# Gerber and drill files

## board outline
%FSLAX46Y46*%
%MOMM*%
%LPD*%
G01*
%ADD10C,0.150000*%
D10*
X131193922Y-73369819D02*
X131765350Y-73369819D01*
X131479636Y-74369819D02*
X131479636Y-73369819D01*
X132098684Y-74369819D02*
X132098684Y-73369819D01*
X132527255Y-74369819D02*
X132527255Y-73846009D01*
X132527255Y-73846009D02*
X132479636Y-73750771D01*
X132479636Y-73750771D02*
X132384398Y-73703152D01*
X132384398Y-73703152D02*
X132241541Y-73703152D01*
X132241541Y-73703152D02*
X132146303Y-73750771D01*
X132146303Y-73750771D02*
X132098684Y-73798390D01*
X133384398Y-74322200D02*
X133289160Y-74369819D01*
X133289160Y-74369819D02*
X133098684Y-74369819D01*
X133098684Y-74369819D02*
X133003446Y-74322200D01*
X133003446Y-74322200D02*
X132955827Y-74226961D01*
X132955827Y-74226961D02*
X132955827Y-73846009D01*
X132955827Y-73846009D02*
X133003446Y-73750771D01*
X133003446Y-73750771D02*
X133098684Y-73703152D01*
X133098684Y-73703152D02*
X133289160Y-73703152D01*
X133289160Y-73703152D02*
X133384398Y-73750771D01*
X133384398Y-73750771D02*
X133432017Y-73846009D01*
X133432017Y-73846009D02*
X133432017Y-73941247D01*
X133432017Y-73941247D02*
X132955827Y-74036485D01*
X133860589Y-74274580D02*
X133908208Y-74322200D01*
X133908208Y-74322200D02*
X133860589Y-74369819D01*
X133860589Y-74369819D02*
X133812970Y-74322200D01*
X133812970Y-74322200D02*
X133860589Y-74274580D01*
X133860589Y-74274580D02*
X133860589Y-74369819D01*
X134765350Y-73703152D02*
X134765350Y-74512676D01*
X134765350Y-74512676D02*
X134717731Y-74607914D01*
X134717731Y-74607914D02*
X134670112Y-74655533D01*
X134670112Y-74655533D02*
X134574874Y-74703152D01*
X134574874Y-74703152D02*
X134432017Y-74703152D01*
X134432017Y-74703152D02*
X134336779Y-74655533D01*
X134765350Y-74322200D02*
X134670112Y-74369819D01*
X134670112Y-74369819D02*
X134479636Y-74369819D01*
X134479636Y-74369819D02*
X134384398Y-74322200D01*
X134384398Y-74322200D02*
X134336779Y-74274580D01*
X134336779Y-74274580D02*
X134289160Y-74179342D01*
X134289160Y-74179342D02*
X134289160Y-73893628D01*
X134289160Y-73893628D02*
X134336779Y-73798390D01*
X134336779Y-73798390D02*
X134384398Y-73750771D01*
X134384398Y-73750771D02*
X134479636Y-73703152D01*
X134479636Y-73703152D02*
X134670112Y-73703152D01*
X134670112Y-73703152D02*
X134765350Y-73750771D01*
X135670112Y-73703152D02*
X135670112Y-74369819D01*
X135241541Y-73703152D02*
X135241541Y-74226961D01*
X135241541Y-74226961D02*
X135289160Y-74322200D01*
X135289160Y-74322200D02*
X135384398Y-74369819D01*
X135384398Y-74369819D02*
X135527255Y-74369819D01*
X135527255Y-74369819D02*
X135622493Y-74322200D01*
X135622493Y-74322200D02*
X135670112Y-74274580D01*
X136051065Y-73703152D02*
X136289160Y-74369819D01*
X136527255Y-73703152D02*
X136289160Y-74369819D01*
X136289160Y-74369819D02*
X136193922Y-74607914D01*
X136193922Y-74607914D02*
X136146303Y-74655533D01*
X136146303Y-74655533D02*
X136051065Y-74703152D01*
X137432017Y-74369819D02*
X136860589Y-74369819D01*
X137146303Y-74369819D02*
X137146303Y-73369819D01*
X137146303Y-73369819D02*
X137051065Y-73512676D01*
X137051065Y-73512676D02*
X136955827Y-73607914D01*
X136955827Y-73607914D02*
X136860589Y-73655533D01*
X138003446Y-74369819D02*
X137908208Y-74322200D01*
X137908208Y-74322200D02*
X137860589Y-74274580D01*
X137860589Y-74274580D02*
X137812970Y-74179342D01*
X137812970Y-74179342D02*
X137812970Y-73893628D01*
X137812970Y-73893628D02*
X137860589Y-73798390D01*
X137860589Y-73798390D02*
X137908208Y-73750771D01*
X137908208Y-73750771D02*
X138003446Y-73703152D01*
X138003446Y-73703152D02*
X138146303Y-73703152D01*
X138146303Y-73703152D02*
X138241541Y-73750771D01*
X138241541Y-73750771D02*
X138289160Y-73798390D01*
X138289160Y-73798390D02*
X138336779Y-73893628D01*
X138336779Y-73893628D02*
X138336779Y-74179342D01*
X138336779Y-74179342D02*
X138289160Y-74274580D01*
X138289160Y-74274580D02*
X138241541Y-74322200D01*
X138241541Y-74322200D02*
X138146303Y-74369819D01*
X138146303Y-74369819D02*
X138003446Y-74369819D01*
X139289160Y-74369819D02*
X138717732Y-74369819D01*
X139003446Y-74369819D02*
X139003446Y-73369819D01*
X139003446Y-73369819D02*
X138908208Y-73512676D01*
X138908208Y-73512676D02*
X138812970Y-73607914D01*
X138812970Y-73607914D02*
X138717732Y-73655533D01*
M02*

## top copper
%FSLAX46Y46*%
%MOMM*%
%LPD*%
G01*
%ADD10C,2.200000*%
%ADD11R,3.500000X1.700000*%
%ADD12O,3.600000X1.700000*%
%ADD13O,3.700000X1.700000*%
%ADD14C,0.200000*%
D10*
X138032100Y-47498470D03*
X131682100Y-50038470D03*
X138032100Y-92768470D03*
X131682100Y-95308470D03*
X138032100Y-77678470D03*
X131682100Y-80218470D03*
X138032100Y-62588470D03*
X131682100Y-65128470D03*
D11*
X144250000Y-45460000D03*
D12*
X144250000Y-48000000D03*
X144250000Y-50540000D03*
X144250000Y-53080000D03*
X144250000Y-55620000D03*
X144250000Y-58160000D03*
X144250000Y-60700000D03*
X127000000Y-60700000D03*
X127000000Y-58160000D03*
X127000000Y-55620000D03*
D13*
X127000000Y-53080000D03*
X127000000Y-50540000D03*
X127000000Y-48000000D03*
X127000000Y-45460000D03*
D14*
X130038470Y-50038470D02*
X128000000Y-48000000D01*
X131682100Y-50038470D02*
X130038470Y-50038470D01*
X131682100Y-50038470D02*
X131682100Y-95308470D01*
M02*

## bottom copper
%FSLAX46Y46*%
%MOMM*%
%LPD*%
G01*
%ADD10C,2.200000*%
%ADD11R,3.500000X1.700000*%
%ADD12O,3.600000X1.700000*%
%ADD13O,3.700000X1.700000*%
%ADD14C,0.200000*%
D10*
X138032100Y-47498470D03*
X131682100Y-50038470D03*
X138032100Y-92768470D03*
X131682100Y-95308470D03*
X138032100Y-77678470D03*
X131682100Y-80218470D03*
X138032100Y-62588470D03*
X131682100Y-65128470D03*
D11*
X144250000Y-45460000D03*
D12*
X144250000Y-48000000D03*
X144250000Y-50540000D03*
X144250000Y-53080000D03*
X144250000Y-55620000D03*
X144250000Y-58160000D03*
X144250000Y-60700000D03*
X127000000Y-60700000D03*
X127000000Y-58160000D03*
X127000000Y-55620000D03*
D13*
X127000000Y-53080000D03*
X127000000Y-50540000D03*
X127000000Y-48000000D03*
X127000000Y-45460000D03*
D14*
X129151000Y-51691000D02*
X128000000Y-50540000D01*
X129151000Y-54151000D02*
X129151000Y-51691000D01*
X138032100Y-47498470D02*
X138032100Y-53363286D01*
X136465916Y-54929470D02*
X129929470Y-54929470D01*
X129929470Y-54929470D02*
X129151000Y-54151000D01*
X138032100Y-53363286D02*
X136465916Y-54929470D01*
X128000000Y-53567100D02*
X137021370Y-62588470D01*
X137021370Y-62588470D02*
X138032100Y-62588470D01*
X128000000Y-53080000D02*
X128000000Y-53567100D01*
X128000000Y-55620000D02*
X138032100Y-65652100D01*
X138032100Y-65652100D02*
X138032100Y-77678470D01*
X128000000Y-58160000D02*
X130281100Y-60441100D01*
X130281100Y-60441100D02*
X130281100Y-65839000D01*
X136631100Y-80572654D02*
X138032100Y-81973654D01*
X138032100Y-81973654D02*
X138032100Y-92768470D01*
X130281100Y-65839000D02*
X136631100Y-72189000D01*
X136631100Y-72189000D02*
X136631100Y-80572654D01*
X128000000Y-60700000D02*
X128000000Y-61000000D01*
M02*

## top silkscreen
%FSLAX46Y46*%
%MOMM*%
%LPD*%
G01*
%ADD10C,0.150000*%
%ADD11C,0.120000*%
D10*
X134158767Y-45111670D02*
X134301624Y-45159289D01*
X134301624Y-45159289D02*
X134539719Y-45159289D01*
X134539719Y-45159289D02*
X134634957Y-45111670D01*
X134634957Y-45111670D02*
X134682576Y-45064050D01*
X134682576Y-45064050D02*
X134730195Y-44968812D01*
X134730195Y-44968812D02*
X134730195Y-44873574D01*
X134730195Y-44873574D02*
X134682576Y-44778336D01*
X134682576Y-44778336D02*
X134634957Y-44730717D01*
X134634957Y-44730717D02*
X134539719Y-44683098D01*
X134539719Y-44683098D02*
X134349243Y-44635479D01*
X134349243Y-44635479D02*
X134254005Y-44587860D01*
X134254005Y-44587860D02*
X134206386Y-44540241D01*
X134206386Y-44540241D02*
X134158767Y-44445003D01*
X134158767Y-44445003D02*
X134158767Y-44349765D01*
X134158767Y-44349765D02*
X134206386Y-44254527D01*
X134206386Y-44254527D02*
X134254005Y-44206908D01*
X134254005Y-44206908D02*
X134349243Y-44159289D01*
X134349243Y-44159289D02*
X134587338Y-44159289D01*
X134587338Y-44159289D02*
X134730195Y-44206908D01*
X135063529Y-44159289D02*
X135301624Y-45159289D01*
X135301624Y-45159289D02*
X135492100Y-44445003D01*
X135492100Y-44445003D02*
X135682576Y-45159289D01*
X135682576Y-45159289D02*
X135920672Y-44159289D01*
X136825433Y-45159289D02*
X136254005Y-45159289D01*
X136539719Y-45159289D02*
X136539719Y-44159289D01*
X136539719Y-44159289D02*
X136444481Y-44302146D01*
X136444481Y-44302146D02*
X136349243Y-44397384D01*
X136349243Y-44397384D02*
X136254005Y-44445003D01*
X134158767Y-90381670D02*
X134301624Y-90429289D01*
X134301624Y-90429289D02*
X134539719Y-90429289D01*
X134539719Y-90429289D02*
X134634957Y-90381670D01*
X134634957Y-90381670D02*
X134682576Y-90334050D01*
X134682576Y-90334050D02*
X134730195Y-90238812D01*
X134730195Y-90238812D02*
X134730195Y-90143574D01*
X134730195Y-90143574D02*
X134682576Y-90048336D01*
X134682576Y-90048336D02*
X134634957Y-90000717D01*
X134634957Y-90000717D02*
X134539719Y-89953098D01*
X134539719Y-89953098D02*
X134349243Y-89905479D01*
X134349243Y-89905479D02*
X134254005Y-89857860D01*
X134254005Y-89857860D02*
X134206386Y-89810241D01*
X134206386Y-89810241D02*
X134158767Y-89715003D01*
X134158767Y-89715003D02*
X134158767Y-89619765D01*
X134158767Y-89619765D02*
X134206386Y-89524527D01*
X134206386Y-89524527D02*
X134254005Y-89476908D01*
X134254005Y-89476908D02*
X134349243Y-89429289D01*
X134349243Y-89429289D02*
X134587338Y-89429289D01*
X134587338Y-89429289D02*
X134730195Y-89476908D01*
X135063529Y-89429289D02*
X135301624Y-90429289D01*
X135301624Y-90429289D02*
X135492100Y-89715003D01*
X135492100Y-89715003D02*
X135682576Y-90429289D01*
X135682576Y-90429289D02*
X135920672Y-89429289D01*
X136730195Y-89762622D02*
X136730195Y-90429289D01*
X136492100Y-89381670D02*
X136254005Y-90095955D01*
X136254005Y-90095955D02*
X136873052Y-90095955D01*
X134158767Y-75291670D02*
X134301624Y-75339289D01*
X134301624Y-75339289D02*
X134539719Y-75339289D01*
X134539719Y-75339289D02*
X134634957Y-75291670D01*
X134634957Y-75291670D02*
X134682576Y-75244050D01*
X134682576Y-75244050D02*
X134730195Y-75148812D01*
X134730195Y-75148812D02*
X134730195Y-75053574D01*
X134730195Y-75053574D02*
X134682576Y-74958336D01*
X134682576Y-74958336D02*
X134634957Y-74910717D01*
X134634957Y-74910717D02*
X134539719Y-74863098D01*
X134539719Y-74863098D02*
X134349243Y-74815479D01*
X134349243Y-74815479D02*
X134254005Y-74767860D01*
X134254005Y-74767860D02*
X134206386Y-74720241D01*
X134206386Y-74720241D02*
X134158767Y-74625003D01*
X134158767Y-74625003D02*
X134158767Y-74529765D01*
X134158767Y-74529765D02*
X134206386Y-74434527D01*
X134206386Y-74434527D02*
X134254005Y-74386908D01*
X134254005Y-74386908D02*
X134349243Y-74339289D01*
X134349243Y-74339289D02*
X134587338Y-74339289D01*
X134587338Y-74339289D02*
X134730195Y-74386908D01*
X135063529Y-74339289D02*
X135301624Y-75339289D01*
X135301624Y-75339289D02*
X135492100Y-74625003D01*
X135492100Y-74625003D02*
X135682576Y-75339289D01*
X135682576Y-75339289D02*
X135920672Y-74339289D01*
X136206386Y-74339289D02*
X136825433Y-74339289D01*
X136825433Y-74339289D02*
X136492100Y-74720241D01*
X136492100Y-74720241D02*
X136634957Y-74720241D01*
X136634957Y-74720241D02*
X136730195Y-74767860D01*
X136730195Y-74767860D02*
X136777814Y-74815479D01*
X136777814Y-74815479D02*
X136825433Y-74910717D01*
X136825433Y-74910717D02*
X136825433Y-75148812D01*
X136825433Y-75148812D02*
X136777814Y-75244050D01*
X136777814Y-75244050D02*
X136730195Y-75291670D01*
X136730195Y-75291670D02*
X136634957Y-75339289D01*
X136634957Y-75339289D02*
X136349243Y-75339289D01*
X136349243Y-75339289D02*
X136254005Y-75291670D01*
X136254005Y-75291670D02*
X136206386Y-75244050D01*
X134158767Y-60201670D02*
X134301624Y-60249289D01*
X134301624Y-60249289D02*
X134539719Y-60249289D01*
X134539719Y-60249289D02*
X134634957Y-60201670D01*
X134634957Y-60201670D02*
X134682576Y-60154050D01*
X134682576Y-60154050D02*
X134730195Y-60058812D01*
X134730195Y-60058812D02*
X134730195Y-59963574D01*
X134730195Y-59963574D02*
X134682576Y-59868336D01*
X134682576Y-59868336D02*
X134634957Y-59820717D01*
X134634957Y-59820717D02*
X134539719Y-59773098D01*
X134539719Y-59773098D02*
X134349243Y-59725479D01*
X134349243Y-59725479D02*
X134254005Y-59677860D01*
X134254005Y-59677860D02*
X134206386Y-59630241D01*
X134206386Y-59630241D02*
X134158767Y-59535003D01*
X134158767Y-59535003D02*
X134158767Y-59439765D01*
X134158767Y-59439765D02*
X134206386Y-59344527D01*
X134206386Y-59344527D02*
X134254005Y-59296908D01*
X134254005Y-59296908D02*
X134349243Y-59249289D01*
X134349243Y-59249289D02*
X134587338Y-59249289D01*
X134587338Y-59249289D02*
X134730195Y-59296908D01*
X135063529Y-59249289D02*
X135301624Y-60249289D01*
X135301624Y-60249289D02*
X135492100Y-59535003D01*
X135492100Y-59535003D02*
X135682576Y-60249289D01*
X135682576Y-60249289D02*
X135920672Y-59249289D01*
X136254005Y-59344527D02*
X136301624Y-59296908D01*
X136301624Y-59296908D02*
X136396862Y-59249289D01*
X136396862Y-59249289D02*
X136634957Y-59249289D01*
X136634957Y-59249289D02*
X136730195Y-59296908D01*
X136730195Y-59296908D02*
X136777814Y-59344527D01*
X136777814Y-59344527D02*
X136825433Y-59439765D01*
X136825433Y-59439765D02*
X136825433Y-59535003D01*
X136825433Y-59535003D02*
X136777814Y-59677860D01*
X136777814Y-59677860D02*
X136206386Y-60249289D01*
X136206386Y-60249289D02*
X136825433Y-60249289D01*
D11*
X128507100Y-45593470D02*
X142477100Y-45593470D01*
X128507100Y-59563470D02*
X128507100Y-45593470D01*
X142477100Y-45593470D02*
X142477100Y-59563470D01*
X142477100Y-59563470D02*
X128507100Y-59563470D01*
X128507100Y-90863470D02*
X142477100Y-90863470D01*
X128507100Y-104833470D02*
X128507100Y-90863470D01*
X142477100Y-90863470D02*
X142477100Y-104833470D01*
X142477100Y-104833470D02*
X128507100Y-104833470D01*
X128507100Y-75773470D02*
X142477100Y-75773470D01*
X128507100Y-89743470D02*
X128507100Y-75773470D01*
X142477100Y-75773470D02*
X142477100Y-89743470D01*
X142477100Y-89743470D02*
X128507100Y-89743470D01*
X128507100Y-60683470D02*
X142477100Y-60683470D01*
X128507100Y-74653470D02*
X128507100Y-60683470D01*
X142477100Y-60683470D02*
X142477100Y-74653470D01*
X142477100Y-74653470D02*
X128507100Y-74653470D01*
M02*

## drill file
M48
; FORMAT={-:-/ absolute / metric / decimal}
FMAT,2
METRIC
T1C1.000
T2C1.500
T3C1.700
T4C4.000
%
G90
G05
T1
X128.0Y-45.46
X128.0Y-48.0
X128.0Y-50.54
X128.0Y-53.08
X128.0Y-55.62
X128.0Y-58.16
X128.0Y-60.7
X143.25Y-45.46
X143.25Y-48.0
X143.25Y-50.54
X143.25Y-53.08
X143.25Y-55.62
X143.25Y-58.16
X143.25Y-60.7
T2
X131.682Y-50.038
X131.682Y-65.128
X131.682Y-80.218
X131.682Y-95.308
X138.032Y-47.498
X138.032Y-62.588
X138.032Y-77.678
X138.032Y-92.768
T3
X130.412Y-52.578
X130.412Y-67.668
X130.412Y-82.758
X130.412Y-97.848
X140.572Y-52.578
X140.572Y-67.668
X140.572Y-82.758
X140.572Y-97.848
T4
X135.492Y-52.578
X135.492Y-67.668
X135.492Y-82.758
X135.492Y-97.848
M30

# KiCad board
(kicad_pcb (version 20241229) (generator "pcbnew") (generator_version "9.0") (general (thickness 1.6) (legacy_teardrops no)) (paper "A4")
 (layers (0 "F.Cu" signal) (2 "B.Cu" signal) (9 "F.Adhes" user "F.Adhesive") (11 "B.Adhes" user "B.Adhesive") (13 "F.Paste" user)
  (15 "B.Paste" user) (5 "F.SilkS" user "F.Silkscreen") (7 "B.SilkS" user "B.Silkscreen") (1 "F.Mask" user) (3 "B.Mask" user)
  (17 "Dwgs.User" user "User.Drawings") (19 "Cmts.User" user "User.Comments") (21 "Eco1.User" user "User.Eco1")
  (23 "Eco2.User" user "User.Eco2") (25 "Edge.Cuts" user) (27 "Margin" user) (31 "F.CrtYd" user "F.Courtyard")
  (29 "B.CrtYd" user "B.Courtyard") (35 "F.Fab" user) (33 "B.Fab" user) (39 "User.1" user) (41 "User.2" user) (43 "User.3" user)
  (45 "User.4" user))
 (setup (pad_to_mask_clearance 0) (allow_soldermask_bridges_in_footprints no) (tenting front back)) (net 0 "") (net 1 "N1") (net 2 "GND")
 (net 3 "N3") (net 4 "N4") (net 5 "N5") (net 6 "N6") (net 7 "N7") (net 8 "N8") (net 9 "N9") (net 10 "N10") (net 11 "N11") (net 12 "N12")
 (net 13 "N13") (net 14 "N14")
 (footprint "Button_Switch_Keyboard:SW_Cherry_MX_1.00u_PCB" (layer "F.Cu") (at 138.0321 47.49847)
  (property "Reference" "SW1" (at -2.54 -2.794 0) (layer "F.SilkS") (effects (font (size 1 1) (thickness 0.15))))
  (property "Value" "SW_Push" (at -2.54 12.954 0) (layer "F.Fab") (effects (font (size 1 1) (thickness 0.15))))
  (fp_line (start -9.525 -1.905) (end 4.445 -1.905) (stroke (width 0.12) (type solid)) (layer "F.SilkS"))
  (fp_line (start -9.525 12.065) (end -9.525 -1.905) (stroke (width 0.12) (type solid)) (layer "F.SilkS"))
  (fp_line (start 4.445 -1.905) (end 4.445 12.065) (stroke (width 0.12) (type solid)) (layer "F.SilkS"))
  (fp_line (start 4.445 12.065) (end -9.525 12.065) (stroke (width 0.12) (type solid)) (layer "F.SilkS"))
  (pad "" np_thru_hole circle (at -7.62 5.08) (size 1.7 1.7) (drill 1.7) (layers "*.Cu" "*.Mask"))
  (pad "" np_thru_hole circle (at -2.54 5.08) (size 4 4) (drill 4) (layers "*.Cu" "*.Mask"))
  (pad "" np_thru_hole circle (at 2.54 5.08) (size 1.7 1.7) (drill 1.7) (layers "*.Cu" "*.Mask"))
  (pad "1" thru_hole circle (at 0 0) (size 2.2 2.2) (drill 1.5) (layers "*.Cu" "*.Mask") (remove_unused_layers no) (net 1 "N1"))
  (pad "2" thru_hole circle (at -6.35 2.54) (size 2.2 2.2) (drill 1.5) (layers "*.Cu" "*.Mask") (remove_unused_layers no) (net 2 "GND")))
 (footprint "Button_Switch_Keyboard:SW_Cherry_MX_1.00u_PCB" (layer "F.Cu") (at 138.0321 92.76847)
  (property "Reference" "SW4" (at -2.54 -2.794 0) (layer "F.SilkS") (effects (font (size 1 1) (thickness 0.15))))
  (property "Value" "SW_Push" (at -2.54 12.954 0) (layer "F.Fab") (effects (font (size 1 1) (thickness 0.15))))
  (fp_line (start -9.525 -1.905) (end 4.445 -1.905) (stroke (width 0.12) (type solid)) (layer "F.SilkS"))
  (fp_line (start -9.525 12.065) (end -9.525 -1.905) (stroke (width 0.12) (type solid)) (layer "F.SilkS"))
  (fp_line (start 4.445 -1.905) (end 4.445 12.065) (stroke (width 0.12) (type solid)) (layer "F.SilkS"))
  (fp_line (start 4.445 12.065) (end -9.525 12.065) (stroke (width 0.12) (type solid)) (layer "F.SilkS"))
  (pad "" np_thru_hole circle (at -7.62 5.08) (size 1.7 1.7) (drill 1.7) (layers "*.Cu" "*.Mask"))
  (pad "" np_thru_hole circle (at -2.54 5.08) (size 4 4) (drill 4) (layers "*.Cu" "*.Mask"))
  (pad "" np_thru_hole circle (at 2.54 5.08) (size 1.7 1.7) (drill 1.7) (layers "*.Cu" "*.Mask"))
  (pad "1" thru_hole circle (at 0 0) (size 2.2 2.2) (drill 1.5) (layers "*.Cu" "*.Mask") (remove_unused_layers no) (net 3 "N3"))
  (pad "2" thru_hole circle (at -6.35 2.54) (size 2.2 2.2) (drill 1.5) (layers "*.Cu" "*.Mask") (remove_unused_layers no) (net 2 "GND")))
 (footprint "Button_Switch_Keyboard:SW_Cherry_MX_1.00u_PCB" (layer "F.Cu") (at 138.0321 77.67847)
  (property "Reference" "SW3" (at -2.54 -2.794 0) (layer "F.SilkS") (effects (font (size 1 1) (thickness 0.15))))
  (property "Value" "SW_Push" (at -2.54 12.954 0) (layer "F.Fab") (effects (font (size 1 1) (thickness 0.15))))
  (fp_line (start -9.525 -1.905) (end 4.445 -1.905) (stroke (width 0.12) (type solid)) (layer "F.SilkS"))
  (fp_line (start -9.525 12.065) (end -9.525 -1.905) (stroke (width 0.12) (type solid)) (layer "F.SilkS"))
  (fp_line (start 4.445 -1.905) (end 4.445 12.065) (stroke (width 0.12) (type solid)) (layer "F.SilkS"))
  (fp_line (start 4.445 12.065) (end -9.525 12.065) (stroke (width 0.12) (type solid)) (layer "F.SilkS"))
  (pad "" np_thru_hole circle (at -7.62 5.08) (size 1.7 1.7) (drill 1.7) (layers "*.Cu" "*.Mask"))
  (pad "" np_thru_hole circle (at -2.54 5.08) (size 4 4) (drill 4) (layers "*.Cu" "*.Mask"))
  (pad "" np_thru_hole circle (at 2.54 5.08) (size 1.7 1.7) (drill 1.7) (layers "*.Cu" "*.Mask"))
  (pad "1" thru_hole circle (at 0 0) (size 2.2 2.2) (drill 1.5) (layers "*.Cu" "*.Mask") (remove_unused_layers no) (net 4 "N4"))
  (pad "2" thru_hole circle (at -6.35 2.54) (size 2.2 2.2) (drill 1.5) (layers "*.Cu" "*.Mask") (remove_unused_layers no) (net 2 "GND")))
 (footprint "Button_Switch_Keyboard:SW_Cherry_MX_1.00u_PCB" (layer "F.Cu") (at 138.0321 62.58847)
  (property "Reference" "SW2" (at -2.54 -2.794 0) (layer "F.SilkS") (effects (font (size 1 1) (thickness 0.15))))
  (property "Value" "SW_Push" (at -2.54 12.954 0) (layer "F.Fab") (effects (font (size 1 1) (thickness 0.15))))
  (fp_line (start -9.525 -1.905) (end 4.445 -1.905) (stroke (width 0.12) (type solid)) (layer "F.SilkS"))
  (fp_line (start -9.525 12.065) (end -9.525 -1.905) (stroke (width 0.12) (type solid)) (layer "F.SilkS"))
  (fp_line (start 4.445 -1.905) (end 4.445 12.065) (stroke (width 0.12) (type solid)) (layer "F.SilkS"))
  (fp_line (start 4.445 12.065) (end -9.525 12.065) (stroke (width 0.12) (type solid)) (layer "F.SilkS"))
  (pad "" np_thru_hole circle (at -7.62 5.08) (size 1.7 1.7) (drill 1.7) (layers "*.Cu" "*.Mask"))
  (pad "" np_thru_hole circle (at -2.54 5.08) (size 4 4) (drill 4) (layers "*.Cu" "*.Mask"))
  (pad "" np_thru_hole circle (at 2.54 5.08) (size 1.7 1.7) (drill 1.7) (layers "*.Cu" "*.Mask"))
  (pad "1" thru_hole circle (at 0 0) (size 2.2 2.2) (drill 1.5) (layers "*.Cu" "*.Mask") (remove_unused_layers no) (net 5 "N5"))
  (pad "2" thru_hole circle (at -6.35 2.54) (size 2.2 2.2) (drill 1.5) (layers "*.Cu" "*.Mask") (remove_unused_layers no) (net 2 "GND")))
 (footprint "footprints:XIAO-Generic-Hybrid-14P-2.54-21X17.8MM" (layer "B.Cu") (at 135.625 53.08 180)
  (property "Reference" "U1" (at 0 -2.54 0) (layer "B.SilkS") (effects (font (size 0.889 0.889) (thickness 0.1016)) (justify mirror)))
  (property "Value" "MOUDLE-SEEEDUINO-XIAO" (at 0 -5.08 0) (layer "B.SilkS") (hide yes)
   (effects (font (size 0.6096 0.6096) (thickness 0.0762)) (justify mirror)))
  (pad "1" thru_hole rect (at -7.625 7.62 180) (size 3.5 1.7) (drill 1 (offset -1 0)) (layers "*.Cu" "*.Mask") (remove_unused_layers no)
   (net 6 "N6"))
  (pad "2" thru_hole oval (at -7.625 5.08 180) (size 3.6 1.7) (drill 1 (offset -1 0)) (layers "*.Cu" "*.Mask") (remove_unused_layers no)
   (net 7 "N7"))
  (pad "3" thru_hole oval (at -7.625 2.54 180) (size 3.6 1.7) (drill 1 (offset -1 0)) (layers "*.Cu" "*.Mask") (remove_unused_layers no)
   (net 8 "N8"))
  (pad "4" thru_hole oval (at -7.625 0 180) (size 3.6 1.7) (drill 1 (offset -1 0)) (layers "*.Cu" "*.Mask") (remove_unused_layers no)
   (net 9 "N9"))
  (pad "5" thru_hole oval (at -7.625 -2.54 180) (size 3.6 1.7) (drill 1 (offset -1 0)) (layers "*.Cu" "*.Mask") (remove_unused_layers no)
   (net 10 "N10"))
  (pad "6" thru_hole oval (at -7.625 -5.08) (size 3.6 1.7) (drill 1 (offset 1 0)) (layers "*.Cu" "*.Mask") (remove_unused_layers no)
   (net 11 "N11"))
  (pad "7" thru_hole oval (at -7.625 -7.62 180) (size 3.6 1.7) (drill 1 (offset -1 0)) (layers "*.Cu" "*.Mask") (remove_unused_layers no)
   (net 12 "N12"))
  (pad "8" thru_hole oval (at 7.625 -7.62 180) (size 3.6 1.7) (drill 1 (offset 1 0)) (layers "*.Cu" "*.Mask") (remove_unused_layers no)
   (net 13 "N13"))
  (pad "9" thru_hole oval (at 7.625 -5.08 180) (size 3.6 1.7) (drill 1 (offset 1 0)) (layers "*.Cu" "*.Mask") (remove_unused_layers no)
   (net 3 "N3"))
  (pad "10" thru_hole oval (at 7.625 -2.54 180) (size 3.6 1.7) (drill 1 (offset 1 0)) (layers "*.Cu" "*.Mask") (remove_unused_layers no)
   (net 4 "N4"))
  (pad "11" thru_hole oval (at 7.625 0 180) (size 3.7 1.7) (drill 1 (offset 1 0)) (layers "*.Cu" "*.Mask") (remove_unused_layers no)
   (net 5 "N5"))
  (pad "12" thru_hole oval (at 7.625 2.54 180) (size 3.7 1.7) (drill 1 (offset 1 0)) (layers "*.Cu" "*.Mask") (remove_unused_layers no)
   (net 1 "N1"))
  (pad "13" thru_hole oval (at 7.625 5.08 180) (size 3.7 1.7) (drill 1 (offset 1 0)) (layers "*.Cu" "B.Mask") (remove_unused_layers no)
   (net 2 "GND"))
  (pad "14" thru_hole oval (at 7.625 7.62 180) (size 3.7 1.7) (drill 1 (offset 1 0)) (layers "*.Cu" "*.Mask") (remove_unused_layers no)
   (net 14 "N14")))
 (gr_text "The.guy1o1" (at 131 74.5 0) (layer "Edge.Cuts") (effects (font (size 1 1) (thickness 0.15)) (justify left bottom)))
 (segment (start 129.151 51.691) (end 128 50.54) (width 0.2) (layer "B.Cu") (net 1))
 (segment (start 129.151 54.151) (end 129.151 51.691) (width 0.2) (layer "B.Cu") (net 1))
 (segment (start 138.0321 47.49847) (end 138.0321 53.363286) (width 0.2) (layer "B.Cu") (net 1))
 (segment (start 136.465916 54.92947) (end 129.92947 54.92947) (width 0.2) (layer "B.Cu") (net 1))
 (segment (start 129.92947 54.92947) (end 129.151 54.151) (width 0.2) (layer "B.Cu") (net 1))
 (segment (start 138.0321 53.363286) (end 136.465916 54.92947) (width 0.2) (layer "B.Cu") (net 1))
 (segment (start 130.03847 50.03847) (end 128 48) (width 0.2) (layer "F.Cu") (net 2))
 (segment (start 131.6821 50.03847) (end 130.03847 50.03847) (width 0.2) (layer "F.Cu") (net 2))
 (segment (start 131.6821 50.03847) (end 131.6821 95.30847) (width 0.2) (layer "F.Cu") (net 2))
 (segment (start 128 53.5671) (end 137.02137 62.58847) (width 0.2) (layer "B.Cu") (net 5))
 (segment (start 137.02137 62.58847) (end 138.0321 62.58847) (width 0.2) (layer "B.Cu") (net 5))
 (segment (start 128 53.08) (end 128 53.5671) (width 0.2) (layer "B.Cu") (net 5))
 (segment (start 128 55.62) (end 138.0321 65.6521) (width 0.2) (layer "B.Cu") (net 4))
 (segment (start 138.0321 65.6521) (end 138.0321 77.67847) (width 0.2) (layer "B.Cu") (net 4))
 (segment (start 128 58.16) (end 130.2811 60.4411) (width 0.2) (layer "B.Cu") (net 3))
 (segment (start 130.2811 60.4411) (end 130.2811 65.839) (width 0.2) (layer "B.Cu") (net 3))
 (segment (start 136.6311 80.572654) (end 138.0321 81.973654) (width 0.2) (layer "B.Cu") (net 3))
 (segment (start 138.0321 81.973654) (end 138.0321 92.76847) (width 0.2) (layer "B.Cu") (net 3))
 (segment (start 130.2811 65.839) (end 136.6311 72.189) (width 0.2) (layer "B.Cu") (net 3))
 (segment (start 136.6311 72.189) (end 136.6311 80.572654) (width 0.2) (layer "B.Cu") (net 3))
 (segment (start 128 60.7) (end 128 61) (width 0.2) (layer "B.Cu") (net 13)))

